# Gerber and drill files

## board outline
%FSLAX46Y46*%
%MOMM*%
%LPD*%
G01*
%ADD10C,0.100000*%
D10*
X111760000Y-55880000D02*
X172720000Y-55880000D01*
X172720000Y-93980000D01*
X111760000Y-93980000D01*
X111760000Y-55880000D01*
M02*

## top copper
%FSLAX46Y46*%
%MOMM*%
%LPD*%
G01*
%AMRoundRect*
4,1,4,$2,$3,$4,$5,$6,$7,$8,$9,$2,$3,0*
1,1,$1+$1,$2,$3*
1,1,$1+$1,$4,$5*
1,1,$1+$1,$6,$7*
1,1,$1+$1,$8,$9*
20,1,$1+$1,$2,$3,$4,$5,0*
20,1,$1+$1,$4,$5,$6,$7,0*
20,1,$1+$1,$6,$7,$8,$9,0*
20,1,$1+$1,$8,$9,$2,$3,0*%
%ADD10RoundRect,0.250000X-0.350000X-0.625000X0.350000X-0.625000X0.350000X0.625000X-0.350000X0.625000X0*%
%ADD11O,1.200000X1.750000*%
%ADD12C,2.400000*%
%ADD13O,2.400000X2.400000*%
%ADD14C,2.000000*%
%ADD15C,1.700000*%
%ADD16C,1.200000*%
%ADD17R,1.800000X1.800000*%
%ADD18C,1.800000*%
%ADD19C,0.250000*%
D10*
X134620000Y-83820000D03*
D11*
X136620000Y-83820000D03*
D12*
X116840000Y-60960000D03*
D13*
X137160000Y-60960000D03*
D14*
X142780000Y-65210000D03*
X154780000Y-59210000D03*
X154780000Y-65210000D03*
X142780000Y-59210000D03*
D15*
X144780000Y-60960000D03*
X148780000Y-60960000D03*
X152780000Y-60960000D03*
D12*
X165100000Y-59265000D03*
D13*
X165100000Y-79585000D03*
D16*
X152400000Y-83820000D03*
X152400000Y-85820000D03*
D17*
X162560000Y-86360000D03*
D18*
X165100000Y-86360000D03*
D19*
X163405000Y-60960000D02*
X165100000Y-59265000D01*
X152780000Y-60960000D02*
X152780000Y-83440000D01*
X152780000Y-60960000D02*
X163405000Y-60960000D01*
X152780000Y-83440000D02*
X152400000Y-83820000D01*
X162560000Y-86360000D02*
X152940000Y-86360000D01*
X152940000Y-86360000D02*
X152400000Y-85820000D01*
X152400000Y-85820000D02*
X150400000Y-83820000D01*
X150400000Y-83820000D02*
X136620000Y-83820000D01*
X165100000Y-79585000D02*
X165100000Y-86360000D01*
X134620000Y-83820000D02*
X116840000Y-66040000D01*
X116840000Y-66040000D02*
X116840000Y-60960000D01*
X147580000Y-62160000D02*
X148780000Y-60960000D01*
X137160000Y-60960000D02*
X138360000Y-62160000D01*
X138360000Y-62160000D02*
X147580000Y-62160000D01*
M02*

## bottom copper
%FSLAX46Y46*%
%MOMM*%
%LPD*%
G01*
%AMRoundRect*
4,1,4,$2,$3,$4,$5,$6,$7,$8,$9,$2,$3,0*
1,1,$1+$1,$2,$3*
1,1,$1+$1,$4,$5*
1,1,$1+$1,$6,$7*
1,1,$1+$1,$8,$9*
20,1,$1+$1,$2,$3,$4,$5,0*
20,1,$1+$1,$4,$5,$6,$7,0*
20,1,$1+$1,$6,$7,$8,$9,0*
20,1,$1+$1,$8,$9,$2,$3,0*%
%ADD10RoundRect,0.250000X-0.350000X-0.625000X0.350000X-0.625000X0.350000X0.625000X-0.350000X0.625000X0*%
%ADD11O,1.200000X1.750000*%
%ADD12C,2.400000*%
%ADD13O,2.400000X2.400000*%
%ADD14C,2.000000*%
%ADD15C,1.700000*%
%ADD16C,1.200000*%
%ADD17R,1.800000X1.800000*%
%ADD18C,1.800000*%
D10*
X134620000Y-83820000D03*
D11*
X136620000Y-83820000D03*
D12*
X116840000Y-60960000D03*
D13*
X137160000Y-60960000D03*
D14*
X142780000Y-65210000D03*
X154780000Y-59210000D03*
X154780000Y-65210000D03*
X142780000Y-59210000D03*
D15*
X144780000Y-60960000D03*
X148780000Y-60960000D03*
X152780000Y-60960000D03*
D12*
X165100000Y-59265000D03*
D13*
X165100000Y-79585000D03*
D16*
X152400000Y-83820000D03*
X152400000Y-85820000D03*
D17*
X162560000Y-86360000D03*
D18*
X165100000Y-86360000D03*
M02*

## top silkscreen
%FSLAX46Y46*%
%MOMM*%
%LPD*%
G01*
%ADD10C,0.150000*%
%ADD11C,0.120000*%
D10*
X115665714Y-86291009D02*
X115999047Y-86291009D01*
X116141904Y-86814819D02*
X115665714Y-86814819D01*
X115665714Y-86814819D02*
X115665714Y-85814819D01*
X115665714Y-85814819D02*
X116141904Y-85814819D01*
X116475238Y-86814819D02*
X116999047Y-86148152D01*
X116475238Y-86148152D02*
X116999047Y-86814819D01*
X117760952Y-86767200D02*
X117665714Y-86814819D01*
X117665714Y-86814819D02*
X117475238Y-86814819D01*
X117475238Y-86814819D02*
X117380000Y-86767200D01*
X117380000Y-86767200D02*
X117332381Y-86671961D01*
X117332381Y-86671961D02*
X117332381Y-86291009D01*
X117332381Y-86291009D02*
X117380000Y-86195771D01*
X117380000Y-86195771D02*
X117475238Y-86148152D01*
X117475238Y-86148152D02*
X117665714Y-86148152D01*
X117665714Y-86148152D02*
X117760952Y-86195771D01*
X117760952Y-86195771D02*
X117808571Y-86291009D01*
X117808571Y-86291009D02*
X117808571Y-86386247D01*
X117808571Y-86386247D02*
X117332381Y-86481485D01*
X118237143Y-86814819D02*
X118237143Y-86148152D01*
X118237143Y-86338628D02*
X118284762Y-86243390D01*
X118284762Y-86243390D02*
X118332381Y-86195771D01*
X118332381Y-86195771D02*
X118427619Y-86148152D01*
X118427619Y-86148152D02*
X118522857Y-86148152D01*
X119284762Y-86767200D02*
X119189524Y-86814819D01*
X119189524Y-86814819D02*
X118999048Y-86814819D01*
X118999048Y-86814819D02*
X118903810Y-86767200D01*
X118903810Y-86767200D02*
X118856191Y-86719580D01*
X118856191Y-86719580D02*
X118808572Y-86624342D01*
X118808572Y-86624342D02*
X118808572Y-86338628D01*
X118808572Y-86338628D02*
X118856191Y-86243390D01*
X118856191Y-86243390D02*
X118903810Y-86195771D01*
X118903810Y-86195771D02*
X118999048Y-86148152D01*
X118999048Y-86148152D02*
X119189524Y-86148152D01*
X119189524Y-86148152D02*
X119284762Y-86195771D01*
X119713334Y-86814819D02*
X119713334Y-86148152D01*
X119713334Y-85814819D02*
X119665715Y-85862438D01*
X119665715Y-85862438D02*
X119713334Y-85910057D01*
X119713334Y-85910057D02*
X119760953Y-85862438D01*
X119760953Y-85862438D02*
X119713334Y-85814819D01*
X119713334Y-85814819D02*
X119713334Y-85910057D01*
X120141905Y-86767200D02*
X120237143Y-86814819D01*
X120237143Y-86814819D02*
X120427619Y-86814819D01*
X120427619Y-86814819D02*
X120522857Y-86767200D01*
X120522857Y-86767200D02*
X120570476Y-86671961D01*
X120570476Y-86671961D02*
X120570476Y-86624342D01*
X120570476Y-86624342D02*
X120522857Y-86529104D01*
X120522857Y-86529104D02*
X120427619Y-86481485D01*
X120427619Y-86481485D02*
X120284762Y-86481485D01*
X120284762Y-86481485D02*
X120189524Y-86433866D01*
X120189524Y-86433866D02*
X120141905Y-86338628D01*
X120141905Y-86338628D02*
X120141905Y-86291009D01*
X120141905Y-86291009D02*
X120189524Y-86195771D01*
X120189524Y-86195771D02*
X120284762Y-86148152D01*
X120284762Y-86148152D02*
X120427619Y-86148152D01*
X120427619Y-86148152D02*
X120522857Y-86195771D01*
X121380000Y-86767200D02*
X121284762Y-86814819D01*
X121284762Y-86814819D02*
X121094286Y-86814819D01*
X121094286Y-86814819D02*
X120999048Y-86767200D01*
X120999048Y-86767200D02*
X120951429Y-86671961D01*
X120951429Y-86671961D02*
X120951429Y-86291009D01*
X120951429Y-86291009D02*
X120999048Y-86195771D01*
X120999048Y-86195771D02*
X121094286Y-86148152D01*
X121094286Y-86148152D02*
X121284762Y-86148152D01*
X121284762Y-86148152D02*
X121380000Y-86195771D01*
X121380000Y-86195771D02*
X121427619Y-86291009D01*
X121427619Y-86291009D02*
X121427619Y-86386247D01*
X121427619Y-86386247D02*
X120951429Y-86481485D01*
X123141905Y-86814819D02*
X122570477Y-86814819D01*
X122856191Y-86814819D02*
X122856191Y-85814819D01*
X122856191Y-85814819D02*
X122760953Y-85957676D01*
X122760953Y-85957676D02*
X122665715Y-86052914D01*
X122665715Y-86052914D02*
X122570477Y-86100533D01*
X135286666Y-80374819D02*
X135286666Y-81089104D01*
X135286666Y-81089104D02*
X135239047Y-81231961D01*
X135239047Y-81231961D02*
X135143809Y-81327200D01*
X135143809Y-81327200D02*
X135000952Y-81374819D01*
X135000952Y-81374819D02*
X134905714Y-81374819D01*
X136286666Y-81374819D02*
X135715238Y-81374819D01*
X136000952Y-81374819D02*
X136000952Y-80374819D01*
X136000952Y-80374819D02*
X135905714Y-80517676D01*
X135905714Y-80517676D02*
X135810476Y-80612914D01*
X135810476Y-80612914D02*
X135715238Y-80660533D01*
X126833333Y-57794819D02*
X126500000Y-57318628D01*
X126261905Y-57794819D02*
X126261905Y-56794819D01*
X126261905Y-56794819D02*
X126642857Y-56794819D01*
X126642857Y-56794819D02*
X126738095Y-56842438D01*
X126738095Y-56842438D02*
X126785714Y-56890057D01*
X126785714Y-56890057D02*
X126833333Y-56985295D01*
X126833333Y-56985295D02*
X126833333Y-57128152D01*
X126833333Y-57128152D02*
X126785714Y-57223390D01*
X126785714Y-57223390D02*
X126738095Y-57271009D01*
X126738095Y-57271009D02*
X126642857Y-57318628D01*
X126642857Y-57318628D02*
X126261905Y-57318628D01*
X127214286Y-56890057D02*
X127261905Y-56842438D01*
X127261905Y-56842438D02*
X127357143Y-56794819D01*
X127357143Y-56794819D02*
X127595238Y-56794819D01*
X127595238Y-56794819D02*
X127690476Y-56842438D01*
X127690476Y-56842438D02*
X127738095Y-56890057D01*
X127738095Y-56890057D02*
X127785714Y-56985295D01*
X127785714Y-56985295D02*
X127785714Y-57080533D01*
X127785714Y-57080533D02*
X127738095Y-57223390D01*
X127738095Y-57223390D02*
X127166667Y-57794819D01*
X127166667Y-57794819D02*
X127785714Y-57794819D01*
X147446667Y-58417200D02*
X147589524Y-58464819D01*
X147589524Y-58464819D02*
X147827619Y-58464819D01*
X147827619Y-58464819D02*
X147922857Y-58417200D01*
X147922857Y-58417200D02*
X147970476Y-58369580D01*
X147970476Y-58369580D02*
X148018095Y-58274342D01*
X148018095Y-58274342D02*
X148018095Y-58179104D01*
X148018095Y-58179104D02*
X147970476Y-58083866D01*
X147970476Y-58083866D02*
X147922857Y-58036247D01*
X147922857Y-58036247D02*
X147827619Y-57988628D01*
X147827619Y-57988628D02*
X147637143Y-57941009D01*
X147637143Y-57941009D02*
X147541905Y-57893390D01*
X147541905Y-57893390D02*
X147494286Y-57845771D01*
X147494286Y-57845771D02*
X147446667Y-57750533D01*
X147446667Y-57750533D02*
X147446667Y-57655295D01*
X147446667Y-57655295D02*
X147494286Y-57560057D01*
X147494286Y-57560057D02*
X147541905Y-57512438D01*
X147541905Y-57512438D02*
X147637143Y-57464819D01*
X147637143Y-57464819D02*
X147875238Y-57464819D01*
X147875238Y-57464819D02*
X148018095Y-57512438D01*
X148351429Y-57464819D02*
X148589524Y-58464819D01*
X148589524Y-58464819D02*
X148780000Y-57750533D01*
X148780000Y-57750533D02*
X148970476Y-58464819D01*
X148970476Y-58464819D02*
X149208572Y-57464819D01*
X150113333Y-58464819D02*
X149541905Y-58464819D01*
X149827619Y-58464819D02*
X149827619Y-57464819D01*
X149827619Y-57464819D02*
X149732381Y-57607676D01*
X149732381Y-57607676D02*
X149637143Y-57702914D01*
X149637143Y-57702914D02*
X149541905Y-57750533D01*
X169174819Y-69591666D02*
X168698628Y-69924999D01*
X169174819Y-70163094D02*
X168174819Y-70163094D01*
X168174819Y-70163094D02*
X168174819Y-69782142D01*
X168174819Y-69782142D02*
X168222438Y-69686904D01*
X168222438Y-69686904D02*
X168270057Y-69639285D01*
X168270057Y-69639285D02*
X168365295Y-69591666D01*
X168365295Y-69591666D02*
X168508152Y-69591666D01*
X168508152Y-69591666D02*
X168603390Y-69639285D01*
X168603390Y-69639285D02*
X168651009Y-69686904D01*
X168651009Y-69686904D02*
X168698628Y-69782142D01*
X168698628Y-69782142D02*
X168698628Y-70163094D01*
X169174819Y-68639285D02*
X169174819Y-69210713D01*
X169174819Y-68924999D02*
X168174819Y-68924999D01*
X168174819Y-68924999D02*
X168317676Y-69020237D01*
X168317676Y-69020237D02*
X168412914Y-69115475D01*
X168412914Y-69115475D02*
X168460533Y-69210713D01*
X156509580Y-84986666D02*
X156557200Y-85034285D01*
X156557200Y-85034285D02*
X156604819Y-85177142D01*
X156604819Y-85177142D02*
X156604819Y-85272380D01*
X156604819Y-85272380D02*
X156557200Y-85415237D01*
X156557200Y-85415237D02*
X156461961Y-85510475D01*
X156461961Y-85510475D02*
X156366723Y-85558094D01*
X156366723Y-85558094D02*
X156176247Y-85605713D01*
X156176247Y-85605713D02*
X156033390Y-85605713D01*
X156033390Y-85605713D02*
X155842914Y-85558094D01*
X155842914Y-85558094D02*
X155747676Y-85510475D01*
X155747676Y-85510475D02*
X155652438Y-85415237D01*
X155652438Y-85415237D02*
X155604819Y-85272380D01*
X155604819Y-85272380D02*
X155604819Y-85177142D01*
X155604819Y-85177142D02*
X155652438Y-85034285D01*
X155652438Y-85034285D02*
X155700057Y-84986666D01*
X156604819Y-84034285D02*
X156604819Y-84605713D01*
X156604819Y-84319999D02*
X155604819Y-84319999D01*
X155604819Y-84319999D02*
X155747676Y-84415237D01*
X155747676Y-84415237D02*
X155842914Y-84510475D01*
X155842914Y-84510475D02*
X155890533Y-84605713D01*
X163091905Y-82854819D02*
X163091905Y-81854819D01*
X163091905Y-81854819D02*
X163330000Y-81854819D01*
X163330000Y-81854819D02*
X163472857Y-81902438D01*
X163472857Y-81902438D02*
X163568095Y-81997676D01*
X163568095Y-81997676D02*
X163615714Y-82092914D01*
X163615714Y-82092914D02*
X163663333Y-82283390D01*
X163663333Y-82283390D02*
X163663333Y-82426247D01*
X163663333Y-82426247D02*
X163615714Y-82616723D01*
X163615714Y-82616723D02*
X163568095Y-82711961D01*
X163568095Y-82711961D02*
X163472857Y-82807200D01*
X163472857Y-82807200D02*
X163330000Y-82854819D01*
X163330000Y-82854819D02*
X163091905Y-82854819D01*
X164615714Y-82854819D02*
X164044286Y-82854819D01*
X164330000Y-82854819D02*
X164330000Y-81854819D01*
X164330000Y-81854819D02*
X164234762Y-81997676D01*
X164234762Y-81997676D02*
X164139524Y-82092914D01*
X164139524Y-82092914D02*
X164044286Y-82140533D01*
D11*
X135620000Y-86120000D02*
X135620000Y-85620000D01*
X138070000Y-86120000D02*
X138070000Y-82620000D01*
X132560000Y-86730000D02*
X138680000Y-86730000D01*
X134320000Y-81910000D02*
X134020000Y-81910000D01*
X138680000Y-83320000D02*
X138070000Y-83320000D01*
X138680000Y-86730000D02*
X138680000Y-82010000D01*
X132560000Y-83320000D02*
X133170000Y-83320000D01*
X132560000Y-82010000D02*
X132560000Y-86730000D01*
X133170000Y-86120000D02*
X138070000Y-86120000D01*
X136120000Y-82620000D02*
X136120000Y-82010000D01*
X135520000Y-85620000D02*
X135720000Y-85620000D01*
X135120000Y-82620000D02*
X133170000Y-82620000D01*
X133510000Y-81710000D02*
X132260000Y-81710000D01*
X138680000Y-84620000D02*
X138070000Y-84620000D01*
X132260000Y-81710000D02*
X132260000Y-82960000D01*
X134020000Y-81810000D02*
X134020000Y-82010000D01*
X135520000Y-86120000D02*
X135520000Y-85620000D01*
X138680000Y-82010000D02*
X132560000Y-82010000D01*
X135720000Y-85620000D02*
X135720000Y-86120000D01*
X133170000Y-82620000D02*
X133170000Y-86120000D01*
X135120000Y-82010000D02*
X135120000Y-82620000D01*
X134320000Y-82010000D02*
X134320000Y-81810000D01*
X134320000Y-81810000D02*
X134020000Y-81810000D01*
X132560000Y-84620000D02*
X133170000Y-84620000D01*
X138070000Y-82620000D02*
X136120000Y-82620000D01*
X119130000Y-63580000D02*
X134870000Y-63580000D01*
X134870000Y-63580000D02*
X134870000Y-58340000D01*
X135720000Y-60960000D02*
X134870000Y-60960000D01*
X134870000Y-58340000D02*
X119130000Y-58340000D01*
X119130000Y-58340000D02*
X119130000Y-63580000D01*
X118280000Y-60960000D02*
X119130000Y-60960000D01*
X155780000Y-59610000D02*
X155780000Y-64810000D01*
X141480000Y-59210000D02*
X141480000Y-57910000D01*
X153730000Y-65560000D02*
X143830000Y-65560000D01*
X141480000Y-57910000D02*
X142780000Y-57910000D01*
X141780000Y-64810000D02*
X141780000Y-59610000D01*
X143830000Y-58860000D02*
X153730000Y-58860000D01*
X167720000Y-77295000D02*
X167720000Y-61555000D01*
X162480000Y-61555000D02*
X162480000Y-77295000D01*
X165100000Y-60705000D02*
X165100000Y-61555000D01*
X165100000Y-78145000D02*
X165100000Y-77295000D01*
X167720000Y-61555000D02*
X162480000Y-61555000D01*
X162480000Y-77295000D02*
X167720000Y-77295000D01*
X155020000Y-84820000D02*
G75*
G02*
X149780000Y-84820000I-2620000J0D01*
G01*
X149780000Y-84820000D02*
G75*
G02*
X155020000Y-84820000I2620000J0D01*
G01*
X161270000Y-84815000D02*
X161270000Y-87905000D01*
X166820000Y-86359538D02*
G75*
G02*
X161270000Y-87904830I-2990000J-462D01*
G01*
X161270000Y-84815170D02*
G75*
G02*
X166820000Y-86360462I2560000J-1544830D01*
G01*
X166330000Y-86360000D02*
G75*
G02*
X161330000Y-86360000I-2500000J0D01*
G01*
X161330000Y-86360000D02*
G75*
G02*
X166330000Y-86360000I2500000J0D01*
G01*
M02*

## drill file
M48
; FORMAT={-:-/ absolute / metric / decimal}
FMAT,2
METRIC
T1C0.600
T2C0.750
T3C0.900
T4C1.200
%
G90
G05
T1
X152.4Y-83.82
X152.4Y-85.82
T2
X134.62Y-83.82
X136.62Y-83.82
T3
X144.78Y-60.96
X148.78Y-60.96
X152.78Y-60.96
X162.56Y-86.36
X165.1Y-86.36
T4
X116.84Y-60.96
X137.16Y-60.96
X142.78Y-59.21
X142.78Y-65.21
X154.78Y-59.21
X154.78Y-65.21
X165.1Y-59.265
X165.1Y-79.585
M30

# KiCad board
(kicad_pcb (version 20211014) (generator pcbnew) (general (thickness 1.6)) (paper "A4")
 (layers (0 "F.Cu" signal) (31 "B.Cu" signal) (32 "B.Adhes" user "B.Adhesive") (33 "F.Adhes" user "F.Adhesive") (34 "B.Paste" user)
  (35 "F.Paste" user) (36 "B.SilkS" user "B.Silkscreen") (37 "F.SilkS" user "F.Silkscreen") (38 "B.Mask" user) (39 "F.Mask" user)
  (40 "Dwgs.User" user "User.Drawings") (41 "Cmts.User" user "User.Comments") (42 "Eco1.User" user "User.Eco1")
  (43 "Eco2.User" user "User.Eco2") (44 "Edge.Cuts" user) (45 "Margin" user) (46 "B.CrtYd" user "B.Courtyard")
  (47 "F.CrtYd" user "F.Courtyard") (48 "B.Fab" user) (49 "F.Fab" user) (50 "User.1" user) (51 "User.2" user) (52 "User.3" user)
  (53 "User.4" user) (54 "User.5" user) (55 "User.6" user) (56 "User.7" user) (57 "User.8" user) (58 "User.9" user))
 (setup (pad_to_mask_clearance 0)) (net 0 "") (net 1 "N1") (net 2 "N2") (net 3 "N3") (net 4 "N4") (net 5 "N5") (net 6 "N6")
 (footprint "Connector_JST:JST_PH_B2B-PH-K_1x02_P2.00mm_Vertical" (layer "F.Cu") (at 134.62 83.82)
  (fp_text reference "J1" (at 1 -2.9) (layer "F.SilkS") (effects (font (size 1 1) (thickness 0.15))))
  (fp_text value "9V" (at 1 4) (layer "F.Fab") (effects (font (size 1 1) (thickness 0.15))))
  (fp_line (start 1 2.3) (end 1 1.8) (layer "F.SilkS") (width 0.12))
  (fp_line (start 3.45 2.3) (end 3.45 -1.2) (layer "F.SilkS") (width 0.12))
  (fp_line (start -2.06 2.91) (end 4.06 2.91) (layer "F.SilkS") (width 0.12))
  (fp_line (start -0.3 -1.91) (end -0.6 -1.91) (layer "F.SilkS") (width 0.12))
  (fp_line (start 4.06 -0.5) (end 3.45 -0.5) (layer "F.SilkS") (width 0.12))
  (fp_line (start 4.06 2.91) (end 4.06 -1.81) (layer "F.SilkS") (width 0.12))
  (fp_line (start -2.06 -0.5) (end -1.45 -0.5) (layer "F.SilkS") (width 0.12))
  (fp_line (start -2.06 -1.81) (end -2.06 2.91) (layer "F.SilkS") (width 0.12))
  (fp_line (start -1.45 2.3) (end 3.45 2.3) (layer "F.SilkS") (width 0.12))
  (fp_line (start 1.5 -1.2) (end 1.5 -1.81) (layer "F.SilkS") (width 0.12))
  (fp_line (start 0.9 1.8) (end 1.1 1.8) (layer "F.SilkS") (width 0.12))
  (fp_line (start 0.5 -1.2) (end -1.45 -1.2) (layer "F.SilkS") (width 0.12))
  (fp_line (start -1.11 -2.11) (end -2.36 -2.11) (layer "F.SilkS") (width 0.12))
  (fp_line (start 4.06 0.8) (end 3.45 0.8) (layer "F.SilkS") (width 0.12))
  (fp_line (start -2.36 -2.11) (end -2.36 -0.86) (layer "F.SilkS") (width 0.12))
  (fp_line (start -0.6 -2.01) (end -0.6 -1.81) (layer "F.SilkS") (width 0.12))
  (fp_line (start 0.9 2.3) (end 0.9 1.8) (layer "F.SilkS") (width 0.12))
  (fp_line (start 4.06 -1.81) (end -2.06 -1.81) (layer "F.SilkS") (width 0.12))
  (fp_line (start 1.1 1.8) (end 1.1 2.3) (layer "F.SilkS") (width 0.12))
  (fp_line (start -1.45 -1.2) (end -1.45 2.3) (layer "F.SilkS") (width 0.12))
  (fp_line (start 0.5 -1.81) (end 0.5 -1.2) (layer "F.SilkS") (width 0.12))
  (fp_line (start -0.3 -1.81) (end -0.3 -2.01) (layer "F.SilkS") (width 0.12))
  (fp_line (start -0.3 -2.01) (end -0.6 -2.01) (layer "F.SilkS") (width 0.12))
  (fp_line (start -2.06 0.8) (end -1.45 0.8) (layer "F.SilkS") (width 0.12))
  (fp_line (start 3.45 -1.2) (end 1.5 -1.2) (layer "F.SilkS") (width 0.12))
  (pad "1" thru_hole roundrect (at 0 0) (size 1.2 1.75) (drill 0.75) (layers *.Cu *.Mask) (roundrect_rratio 0.208333) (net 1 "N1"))
  (pad "2" thru_hole oval (at 2 0) (size 1.2 1.75) (drill 0.75) (layers *.Cu *.Mask) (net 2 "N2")))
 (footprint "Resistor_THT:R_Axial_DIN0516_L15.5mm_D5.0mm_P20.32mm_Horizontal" (layer "F.Cu") (at 116.84 60.96)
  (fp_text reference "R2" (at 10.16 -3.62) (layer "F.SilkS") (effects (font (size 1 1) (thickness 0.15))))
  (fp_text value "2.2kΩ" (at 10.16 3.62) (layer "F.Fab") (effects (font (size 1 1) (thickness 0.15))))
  (fp_line (start 2.29 2.62) (end 18.03 2.62) (layer "F.SilkS") (width 0.12))
  (fp_line (start 18.03 2.62) (end 18.03 -2.62) (layer "F.SilkS") (width 0.12))
  (fp_line (start 18.88 0) (end 18.03 0) (layer "F.SilkS") (width 0.12))
  (fp_line (start 18.03 -2.62) (end 2.29 -2.62) (layer "F.SilkS") (width 0.12))
  (fp_line (start 2.29 -2.62) (end 2.29 2.62) (layer "F.SilkS") (width 0.12))
  (fp_line (start 1.44 0) (end 2.29 0) (layer "F.SilkS") (width 0.12))
  (pad "1" thru_hole circle (at 0 0) (size 2.4 2.4) (drill 1.2) (layers *.Cu *.Mask) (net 1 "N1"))
  (pad "2" thru_hole oval (at 20.32 0) (size 2.4 2.4) (drill 1.2) (layers *.Cu *.Mask) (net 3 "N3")))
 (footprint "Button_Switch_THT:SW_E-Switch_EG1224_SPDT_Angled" (layer "F.Cu") (at 144.78 60.96)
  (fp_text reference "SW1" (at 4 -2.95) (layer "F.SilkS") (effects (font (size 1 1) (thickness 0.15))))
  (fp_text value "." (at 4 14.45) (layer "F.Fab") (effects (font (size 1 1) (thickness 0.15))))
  (fp_line (start 11 -1.35) (end 11 3.85) (layer "F.SilkS") (width 0.12))
  (fp_line (start -3.3 -1.75) (end -3.3 -3.05) (layer "F.SilkS") (width 0.12))
  (fp_line (start 8.95 4.6) (end -0.95 4.6) (layer "F.SilkS") (width 0.12))
  (fp_line (start -3.3 -3.05) (end -2 -3.05) (layer "F.SilkS") (width 0.12))
  (fp_line (start -3 3.85) (end -3 -1.35) (layer "F.SilkS") (width 0.12))
  (fp_line (start -0.95 -2.1) (end 8.95 -2.1) (layer "F.SilkS") (width 0.12))
  (pad "" thru_hole circle (at -2 4.25) (size 2 2) (drill 1.2) (layers *.Cu *.Mask))
  (pad "" thru_hole circle (at 10 -1.75) (size 2 2) (drill 1.2) (layers *.Cu *.Mask))
  (pad "" thru_hole circle (at 10 4.25) (size 2 2) (drill 1.2) (layers *.Cu *.Mask))
  (pad "" thru_hole circle (at -2 -1.75) (size 2 2) (drill 1.2) (layers *.Cu *.Mask))
  (pad "1" thru_hole circle (at 0 0) (size 1.7 1.7) (drill 0.9) (layers *.Cu *.Mask) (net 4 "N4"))
  (pad "2" thru_hole circle (at 4 0) (size 1.7 1.7) (drill 0.9) (layers *.Cu *.Mask) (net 3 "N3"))
  (pad "3" thru_hole circle (at 8 0) (size 1.7 1.7) (drill 0.9) (layers *.Cu *.Mask) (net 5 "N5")))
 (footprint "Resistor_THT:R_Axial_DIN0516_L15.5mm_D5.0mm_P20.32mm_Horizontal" (layer "F.Cu") (at 165.1 59.265 -90)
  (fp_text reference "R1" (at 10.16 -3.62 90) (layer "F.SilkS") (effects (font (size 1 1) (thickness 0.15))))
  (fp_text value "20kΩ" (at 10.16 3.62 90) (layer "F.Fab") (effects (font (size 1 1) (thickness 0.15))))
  (fp_line (start 18.03 -2.62) (end 2.29 -2.62) (layer "F.SilkS") (width 0.12))
  (fp_line (start 2.29 2.62) (end 18.03 2.62) (layer "F.SilkS") (width 0.12))
  (fp_line (start 1.44 0) (end 2.29 0) (layer "F.SilkS") (width 0.12))
  (fp_line (start 18.88 0) (end 18.03 0) (layer "F.SilkS") (width 0.12))
  (fp_line (start 2.29 -2.62) (end 2.29 2.62) (layer "F.SilkS") (width 0.12))
  (fp_line (start 18.03 2.62) (end 18.03 -2.62) (layer "F.SilkS") (width 0.12))
  (pad "1" thru_hole circle (at 0 0 270) (size 2.4 2.4) (drill 1.2) (layers *.Cu *.Mask) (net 5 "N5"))
  (pad "2" thru_hole oval (at 20.32 0 270) (size 2.4 2.4) (drill 1.2) (layers *.Cu *.Mask) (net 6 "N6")))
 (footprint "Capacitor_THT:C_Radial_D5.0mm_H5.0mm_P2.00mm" (layer "F.Cu") (at 152.4 83.82 -90)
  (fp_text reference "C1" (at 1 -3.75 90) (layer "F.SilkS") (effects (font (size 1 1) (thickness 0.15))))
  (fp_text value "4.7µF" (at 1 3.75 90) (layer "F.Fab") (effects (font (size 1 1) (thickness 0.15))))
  (fp_circle (center 1 0) (end 3.62 0) (layer "F.SilkS") (width 0.12) (fill none))
  (pad "1" thru_hole circle (at 0 0 270) (size 1.2 1.2) (drill 0.6) (layers *.Cu *.Mask) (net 5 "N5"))
  (pad "2" thru_hole circle (at 2 0 270) (size 1.2 1.2) (drill 0.6) (layers *.Cu *.Mask) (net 2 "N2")))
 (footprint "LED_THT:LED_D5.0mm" (layer "F.Cu") (at 162.56 86.36)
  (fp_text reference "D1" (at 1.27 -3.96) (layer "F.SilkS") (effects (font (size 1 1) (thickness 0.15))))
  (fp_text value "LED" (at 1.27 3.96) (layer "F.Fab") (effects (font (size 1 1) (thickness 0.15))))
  (fp_line (start -1.29 -1.545) (end -1.29 1.545) (layer "F.SilkS") (width 0.12))
  (fp_arc (start 4.26 -0.000462) (mid 2.072002 2.880433) (end -1.29 1.54483) (layer "F.SilkS") (width 0.12))
  (fp_arc (start -1.29 -1.54483) (mid 2.072002 -2.880433) (end 4.26 0.000462) (layer "F.SilkS") (width 0.12))
  (fp_circle (center 1.27 0) (end 3.77 0) (layer "F.SilkS") (width 0.12) (fill none))
  (pad "1" thru_hole rect (at 0 0) (size 1.8 1.8) (drill 0.9) (layers *.Cu *.Mask) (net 2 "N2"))
  (pad "2" thru_hole circle (at 2.54 0) (size 1.8 1.8) (drill 0.9) (layers *.Cu *.Mask) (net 6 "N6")))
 (gr_rect (start 111.76 55.88) (end 172.72 93.98) (layer "Edge.Cuts") (width 0.1) (fill none))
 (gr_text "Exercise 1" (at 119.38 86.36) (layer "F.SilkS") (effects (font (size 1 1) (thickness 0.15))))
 (segment (start 163.405 60.96) (end 165.1 59.265) (width 0.25) (layer "F.Cu") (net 5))
 (segment (start 152.78 60.96) (end 152.78 83.44) (width 0.25) (layer "F.Cu") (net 5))
 (segment (start 152.78 60.96) (end 163.405 60.96) (width 0.25) (layer "F.Cu") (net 5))
 (segment (start 152.78 83.44) (end 152.4 83.82) (width 0.25) (layer "F.Cu") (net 5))
 (segment (start 162.56 86.36) (end 152.94 86.36) (width 0.25) (layer "F.Cu") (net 2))
 (segment (start 152.94 86.36) (end 152.4 85.82) (width 0.25) (layer "F.Cu") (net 2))
 (segment (start 152.4 85.82) (end 150.4 83.82) (width 0.25) (layer "F.Cu") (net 2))
 (segment (start 150.4 83.82) (end 136.62 83.82) (width 0.25) (layer "F.Cu") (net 2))
 (segment (start 165.1 79.585) (end 165.1 86.36) (width 0.25) (layer "F.Cu") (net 6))
 (segment (start 134.62 83.82) (end 116.84 66.04) (width 0.25) (layer "F.Cu") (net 1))
 (segment (start 116.84 66.04) (end 116.84 60.96) (width 0.25) (layer "F.Cu") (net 1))
 (segment (start 147.58 62.16) (end 148.78 60.96) (width 0.25) (layer "F.Cu") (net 3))
 (segment (start 137.16 60.96) (end 138.36 62.16) (width 0.25) (layer "F.Cu") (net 3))
 (segment (start 138.36 62.16) (end 147.58 62.16) (width 0.25) (layer "F.Cu") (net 3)))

